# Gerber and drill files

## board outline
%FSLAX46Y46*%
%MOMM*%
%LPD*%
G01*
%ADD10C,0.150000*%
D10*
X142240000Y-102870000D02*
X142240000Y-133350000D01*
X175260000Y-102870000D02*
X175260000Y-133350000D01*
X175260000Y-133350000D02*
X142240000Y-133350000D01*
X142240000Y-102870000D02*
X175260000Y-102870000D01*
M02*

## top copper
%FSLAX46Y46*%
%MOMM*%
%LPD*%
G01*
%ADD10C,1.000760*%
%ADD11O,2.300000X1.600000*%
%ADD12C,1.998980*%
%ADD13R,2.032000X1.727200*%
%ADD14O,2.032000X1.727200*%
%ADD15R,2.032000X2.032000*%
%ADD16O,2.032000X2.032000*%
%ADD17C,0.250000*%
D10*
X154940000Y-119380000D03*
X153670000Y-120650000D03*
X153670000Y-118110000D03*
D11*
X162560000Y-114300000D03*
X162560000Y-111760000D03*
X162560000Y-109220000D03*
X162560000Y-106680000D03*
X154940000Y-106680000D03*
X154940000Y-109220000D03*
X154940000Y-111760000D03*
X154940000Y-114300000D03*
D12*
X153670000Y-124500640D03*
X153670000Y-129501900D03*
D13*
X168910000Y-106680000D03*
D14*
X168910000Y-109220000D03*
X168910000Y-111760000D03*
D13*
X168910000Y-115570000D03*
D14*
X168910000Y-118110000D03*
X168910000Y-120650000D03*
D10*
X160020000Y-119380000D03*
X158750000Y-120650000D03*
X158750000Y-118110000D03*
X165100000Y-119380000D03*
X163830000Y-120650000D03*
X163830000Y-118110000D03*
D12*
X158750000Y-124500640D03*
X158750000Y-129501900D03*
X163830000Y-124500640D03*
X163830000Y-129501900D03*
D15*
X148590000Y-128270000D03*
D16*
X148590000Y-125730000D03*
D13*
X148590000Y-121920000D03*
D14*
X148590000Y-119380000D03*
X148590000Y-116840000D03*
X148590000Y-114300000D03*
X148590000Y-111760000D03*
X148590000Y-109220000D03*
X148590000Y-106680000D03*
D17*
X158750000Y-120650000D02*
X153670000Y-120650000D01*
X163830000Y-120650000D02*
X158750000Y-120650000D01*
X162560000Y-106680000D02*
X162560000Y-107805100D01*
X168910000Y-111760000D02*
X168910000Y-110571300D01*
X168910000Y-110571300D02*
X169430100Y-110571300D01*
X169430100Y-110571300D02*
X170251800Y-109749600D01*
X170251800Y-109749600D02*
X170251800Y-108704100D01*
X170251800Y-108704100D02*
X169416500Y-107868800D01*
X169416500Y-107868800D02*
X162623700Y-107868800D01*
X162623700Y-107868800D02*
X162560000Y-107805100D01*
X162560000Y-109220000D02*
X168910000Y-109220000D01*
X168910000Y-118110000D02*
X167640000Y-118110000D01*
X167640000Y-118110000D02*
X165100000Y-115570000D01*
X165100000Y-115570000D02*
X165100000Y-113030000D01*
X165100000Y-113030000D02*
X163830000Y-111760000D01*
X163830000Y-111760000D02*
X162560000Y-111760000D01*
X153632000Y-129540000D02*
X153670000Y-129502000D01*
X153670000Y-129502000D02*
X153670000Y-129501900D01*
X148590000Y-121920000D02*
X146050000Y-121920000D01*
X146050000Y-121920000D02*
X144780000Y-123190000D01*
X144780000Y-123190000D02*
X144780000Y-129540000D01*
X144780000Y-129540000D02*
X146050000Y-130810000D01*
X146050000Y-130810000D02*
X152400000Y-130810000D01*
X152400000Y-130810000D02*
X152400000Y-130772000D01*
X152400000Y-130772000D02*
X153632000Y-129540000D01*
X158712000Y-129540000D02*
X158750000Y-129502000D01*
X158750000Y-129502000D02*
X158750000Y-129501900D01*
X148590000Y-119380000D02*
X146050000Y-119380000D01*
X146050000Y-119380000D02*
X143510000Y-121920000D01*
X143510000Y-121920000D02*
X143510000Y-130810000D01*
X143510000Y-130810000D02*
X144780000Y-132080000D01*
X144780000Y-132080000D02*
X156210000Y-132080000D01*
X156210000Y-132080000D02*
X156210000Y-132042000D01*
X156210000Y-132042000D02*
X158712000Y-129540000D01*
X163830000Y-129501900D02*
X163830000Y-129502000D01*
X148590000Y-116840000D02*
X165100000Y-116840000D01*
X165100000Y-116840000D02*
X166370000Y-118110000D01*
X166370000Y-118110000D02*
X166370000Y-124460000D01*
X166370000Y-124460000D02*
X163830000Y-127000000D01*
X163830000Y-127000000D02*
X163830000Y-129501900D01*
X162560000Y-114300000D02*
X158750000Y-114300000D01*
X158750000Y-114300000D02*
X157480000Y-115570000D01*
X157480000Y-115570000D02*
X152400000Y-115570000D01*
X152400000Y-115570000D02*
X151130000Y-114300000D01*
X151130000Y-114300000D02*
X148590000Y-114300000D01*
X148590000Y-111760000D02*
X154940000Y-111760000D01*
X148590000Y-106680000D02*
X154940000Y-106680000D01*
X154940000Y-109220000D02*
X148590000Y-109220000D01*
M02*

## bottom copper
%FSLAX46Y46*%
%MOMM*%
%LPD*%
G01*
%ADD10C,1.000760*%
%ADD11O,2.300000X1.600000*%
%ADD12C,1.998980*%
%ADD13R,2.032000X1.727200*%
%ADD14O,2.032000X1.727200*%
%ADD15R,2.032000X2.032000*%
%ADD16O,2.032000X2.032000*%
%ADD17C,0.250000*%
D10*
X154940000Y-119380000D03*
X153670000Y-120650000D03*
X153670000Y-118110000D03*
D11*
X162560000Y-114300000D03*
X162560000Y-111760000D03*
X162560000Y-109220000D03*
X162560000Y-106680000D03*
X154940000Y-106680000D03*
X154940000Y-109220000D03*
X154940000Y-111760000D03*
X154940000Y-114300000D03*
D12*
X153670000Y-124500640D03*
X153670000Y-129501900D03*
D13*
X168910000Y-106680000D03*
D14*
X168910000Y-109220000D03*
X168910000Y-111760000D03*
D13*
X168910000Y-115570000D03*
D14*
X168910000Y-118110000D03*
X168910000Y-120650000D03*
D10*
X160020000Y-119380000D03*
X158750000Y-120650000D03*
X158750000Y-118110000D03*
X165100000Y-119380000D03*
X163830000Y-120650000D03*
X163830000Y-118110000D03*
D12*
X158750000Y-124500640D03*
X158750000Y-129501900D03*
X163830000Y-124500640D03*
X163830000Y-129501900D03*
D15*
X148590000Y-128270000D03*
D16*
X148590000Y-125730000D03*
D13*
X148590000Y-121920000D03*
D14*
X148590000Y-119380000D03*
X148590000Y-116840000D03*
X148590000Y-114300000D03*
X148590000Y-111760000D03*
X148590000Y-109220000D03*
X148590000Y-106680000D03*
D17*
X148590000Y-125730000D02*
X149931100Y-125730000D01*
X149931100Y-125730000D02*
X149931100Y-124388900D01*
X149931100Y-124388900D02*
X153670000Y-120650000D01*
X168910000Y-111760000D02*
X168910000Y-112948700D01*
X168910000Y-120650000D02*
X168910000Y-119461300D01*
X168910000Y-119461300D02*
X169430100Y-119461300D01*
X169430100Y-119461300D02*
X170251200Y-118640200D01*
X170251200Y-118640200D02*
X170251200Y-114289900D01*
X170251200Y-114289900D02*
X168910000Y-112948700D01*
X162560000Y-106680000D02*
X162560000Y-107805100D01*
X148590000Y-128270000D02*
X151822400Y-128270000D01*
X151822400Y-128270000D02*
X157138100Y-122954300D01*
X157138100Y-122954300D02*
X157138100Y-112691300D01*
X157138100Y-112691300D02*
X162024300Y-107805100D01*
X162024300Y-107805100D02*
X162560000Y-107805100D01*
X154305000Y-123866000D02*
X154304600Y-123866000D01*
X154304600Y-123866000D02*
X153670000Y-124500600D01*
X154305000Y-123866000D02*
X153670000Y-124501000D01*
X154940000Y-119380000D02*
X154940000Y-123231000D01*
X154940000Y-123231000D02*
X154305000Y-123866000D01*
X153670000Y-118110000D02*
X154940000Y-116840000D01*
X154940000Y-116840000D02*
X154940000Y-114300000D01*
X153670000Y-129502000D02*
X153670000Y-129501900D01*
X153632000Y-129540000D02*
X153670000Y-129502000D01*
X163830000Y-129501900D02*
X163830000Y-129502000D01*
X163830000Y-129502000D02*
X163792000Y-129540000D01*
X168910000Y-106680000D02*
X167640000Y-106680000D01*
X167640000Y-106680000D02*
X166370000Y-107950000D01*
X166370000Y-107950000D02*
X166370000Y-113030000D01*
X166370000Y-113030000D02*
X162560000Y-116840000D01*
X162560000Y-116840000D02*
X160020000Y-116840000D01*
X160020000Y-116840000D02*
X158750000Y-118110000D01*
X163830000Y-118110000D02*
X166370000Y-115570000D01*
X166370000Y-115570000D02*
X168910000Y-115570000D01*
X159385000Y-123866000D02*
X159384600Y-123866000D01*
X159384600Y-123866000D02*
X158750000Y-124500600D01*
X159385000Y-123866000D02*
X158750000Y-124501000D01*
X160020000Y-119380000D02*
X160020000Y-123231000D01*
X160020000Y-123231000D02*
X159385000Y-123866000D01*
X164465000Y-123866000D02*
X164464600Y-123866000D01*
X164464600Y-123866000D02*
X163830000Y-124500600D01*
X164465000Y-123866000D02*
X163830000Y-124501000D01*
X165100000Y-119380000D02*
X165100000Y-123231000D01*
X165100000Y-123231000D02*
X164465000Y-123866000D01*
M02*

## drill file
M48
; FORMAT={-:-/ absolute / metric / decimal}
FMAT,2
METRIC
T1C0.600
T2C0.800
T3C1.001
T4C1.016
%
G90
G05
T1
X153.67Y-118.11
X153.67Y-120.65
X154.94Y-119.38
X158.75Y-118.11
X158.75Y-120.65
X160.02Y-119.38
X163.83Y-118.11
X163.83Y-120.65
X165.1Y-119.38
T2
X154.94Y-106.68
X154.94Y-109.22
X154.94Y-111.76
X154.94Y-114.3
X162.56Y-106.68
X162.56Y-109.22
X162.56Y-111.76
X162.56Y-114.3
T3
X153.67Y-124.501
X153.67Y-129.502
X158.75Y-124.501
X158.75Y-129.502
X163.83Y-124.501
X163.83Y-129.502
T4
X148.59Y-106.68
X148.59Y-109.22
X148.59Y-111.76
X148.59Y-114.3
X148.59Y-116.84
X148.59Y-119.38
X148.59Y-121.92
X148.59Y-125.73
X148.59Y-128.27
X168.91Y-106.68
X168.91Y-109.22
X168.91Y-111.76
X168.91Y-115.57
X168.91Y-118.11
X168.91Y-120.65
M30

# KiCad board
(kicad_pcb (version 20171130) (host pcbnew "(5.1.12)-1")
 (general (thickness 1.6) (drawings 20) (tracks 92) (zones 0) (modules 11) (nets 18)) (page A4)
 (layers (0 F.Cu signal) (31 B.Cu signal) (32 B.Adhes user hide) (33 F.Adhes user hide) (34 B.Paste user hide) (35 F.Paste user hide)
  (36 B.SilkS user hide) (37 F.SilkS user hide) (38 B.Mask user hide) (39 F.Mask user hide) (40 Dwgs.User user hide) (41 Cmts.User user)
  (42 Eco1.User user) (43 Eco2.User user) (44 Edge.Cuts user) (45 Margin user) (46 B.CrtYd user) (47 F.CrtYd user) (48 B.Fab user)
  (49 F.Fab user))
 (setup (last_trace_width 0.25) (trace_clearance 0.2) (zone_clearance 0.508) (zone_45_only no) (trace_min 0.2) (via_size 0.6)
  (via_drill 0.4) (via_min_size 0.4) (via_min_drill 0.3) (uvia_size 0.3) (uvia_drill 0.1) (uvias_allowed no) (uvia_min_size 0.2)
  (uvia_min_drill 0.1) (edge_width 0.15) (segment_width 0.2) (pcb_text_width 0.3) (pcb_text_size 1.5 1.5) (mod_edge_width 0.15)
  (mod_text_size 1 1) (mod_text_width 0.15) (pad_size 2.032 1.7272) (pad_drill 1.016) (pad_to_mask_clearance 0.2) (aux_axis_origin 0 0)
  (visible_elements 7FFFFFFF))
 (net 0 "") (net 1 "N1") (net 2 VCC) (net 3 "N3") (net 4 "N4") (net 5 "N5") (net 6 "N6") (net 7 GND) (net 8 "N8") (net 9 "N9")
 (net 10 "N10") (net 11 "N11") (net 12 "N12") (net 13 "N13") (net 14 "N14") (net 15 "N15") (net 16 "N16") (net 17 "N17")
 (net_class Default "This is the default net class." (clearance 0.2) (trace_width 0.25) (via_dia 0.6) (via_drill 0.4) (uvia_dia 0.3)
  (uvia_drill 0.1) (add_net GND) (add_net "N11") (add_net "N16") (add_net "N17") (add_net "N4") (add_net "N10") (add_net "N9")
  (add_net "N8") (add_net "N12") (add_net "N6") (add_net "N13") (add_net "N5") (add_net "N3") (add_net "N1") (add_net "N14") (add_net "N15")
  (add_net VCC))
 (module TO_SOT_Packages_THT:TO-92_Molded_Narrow (layer F.Cu) (at 153.67 118.11 270)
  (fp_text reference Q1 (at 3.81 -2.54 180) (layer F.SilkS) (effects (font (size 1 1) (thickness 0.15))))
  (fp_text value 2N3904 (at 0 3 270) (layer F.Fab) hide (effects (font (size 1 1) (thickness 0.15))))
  (pad 2 thru_hole circle (at 1.27 -1.27) (size 1.00076 1.00076) (drill 0.6) (layers *.Cu *.Mask F.SilkS) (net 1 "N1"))
  (pad 3 thru_hole circle (at 2.54 0) (size 1.00076 1.00076) (drill 0.6) (layers *.Cu *.Mask F.SilkS) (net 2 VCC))
  (pad 1 thru_hole circle (at 0 0) (size 1.00076 1.00076) (drill 0.6) (layers *.Cu *.Mask F.SilkS) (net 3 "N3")))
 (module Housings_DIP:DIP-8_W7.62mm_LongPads (layer F.Cu) (at 162.56 114.3 180)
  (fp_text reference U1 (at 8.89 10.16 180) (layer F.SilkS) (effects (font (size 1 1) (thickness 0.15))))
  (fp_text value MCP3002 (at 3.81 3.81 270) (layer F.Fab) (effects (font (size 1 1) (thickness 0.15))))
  (pad 1 thru_hole oval (at 0 0 180) (size 2.3 1.6) (drill 0.8) (layers *.Cu *.Mask F.SilkS) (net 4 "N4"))
  (pad 2 thru_hole oval (at 0 2.54 180) (size 2.3 1.6) (drill 0.8) (layers *.Cu *.Mask F.SilkS) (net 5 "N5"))
  (pad 3 thru_hole oval (at 0 5.08 180) (size 2.3 1.6) (drill 0.8) (layers *.Cu *.Mask F.SilkS) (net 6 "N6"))
  (pad 4 thru_hole oval (at 0 7.62 180) (size 2.3 1.6) (drill 0.8) (layers *.Cu *.Mask F.SilkS) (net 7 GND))
  (pad 5 thru_hole oval (at 7.62 7.62 180) (size 2.3 1.6) (drill 0.8) (layers *.Cu *.Mask F.SilkS) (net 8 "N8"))
  (pad 6 thru_hole oval (at 7.62 5.08 180) (size 2.3 1.6) (drill 0.8) (layers *.Cu *.Mask F.SilkS) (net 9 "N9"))
  (pad 7 thru_hole oval (at 7.62 2.54 180) (size 2.3 1.6) (drill 0.8) (layers *.Cu *.Mask F.SilkS) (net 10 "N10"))
  (pad 8 thru_hole oval (at 7.62 0 180) (size 2.3 1.6) (drill 0.8) (layers *.Cu *.Mask F.SilkS) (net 3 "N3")))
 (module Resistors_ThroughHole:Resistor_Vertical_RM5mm (layer F.Cu) (at 153.67 127 270)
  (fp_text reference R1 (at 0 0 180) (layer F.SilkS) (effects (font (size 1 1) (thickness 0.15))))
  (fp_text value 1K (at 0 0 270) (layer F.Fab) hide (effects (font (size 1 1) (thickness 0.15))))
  (pad 1 thru_hole circle (at -2.49936 0 270) (size 1.99898 1.99898) (drill 1.00076) (layers *.Cu *.SilkS *.Mask) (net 1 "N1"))
  (pad 2 thru_hole circle (at 2.5019 0 270) (size 1.99898 1.99898) (drill 1.00076) (layers *.Cu *.SilkS *.Mask) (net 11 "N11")))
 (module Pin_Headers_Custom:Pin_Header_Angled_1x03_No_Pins (layer F.Cu) (at 168.91 106.68)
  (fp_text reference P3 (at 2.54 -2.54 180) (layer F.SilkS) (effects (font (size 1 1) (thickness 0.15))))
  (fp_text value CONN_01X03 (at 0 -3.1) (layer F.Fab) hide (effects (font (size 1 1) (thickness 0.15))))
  (pad 1 thru_hole rect (at 0 0) (size 2.032 1.7272) (drill 1.016) (layers *.Cu *.Mask F.SilkS) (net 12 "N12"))
  (pad 2 thru_hole oval (at 0 2.54) (size 2.032 1.7272) (drill 1.016) (layers *.Cu *.Mask F.SilkS) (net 6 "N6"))
  (pad 3 thru_hole oval (at 0 5.08) (size 2.032 1.7272) (drill 1.016) (layers *.Cu *.Mask F.SilkS) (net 7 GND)))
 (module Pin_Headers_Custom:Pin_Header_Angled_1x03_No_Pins (layer F.Cu) (at 168.91 115.57)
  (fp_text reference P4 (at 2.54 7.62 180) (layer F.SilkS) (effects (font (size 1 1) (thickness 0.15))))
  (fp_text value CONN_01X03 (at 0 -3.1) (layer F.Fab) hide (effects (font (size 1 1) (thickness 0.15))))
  (pad 1 thru_hole rect (at 0 0) (size 2.032 1.7272) (drill 1.016) (layers *.Cu *.Mask F.SilkS) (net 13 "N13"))
  (pad 2 thru_hole oval (at 0 2.54) (size 2.032 1.7272) (drill 1.016) (layers *.Cu *.Mask F.SilkS) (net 5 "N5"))
  (pad 3 thru_hole oval (at 0 5.08) (size 2.032 1.7272) (drill 1.016) (layers *.Cu *.Mask F.SilkS) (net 7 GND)))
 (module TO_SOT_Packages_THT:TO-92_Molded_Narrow (layer F.Cu) (at 158.75 118.11 270)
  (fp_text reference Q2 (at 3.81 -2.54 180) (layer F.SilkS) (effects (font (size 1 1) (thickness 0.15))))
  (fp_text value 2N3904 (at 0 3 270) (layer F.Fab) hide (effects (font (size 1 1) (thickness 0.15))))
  (pad 2 thru_hole circle (at 1.27 -1.27) (size 1.00076 1.00076) (drill 0.6) (layers *.Cu *.Mask F.SilkS) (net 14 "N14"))
  (pad 3 thru_hole circle (at 2.54 0) (size 1.00076 1.00076) (drill 0.6) (layers *.Cu *.Mask F.SilkS) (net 2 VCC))
  (pad 1 thru_hole circle (at 0 0) (size 1.00076 1.00076) (drill 0.6) (layers *.Cu *.Mask F.SilkS) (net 12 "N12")))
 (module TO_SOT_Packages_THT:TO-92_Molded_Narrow (layer F.Cu) (at 163.83 118.11 270)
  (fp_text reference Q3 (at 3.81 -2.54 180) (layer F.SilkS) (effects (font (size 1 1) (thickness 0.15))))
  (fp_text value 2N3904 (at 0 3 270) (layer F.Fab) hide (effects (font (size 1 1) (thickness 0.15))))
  (pad 2 thru_hole circle (at 1.27 -1.27) (size 1.00076 1.00076) (drill 0.6) (layers *.Cu *.Mask F.SilkS) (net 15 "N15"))
  (pad 3 thru_hole circle (at 2.54 0) (size 1.00076 1.00076) (drill 0.6) (layers *.Cu *.Mask F.SilkS) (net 2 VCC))
  (pad 1 thru_hole circle (at 0 0) (size 1.00076 1.00076) (drill 0.6) (layers *.Cu *.Mask F.SilkS) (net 13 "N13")))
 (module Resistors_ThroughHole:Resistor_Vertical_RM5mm (layer F.Cu) (at 158.75 127 270)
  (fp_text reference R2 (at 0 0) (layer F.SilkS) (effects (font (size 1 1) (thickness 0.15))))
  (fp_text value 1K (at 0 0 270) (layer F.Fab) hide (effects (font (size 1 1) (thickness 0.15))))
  (pad 1 thru_hole circle (at -2.49936 0 270) (size 1.99898 1.99898) (drill 1.00076) (layers *.Cu *.SilkS *.Mask) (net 14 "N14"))
  (pad 2 thru_hole circle (at 2.5019 0 270) (size 1.99898 1.99898) (drill 1.00076) (layers *.Cu *.SilkS *.Mask) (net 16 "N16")))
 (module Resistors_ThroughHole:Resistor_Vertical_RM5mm (layer F.Cu) (at 163.83 127 270)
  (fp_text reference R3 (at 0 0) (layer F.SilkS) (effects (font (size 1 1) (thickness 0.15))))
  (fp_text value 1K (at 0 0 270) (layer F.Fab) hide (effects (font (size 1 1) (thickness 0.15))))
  (pad 1 thru_hole circle (at -2.49936 0 270) (size 1.99898 1.99898) (drill 1.00076) (layers *.Cu *.SilkS *.Mask) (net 15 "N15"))
  (pad 2 thru_hole circle (at 2.5019 0 270) (size 1.99898 1.99898) (drill 1.00076) (layers *.Cu *.SilkS *.Mask) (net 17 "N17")))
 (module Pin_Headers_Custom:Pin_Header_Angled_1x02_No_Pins (layer F.Cu) (at 148.59 128.27 180)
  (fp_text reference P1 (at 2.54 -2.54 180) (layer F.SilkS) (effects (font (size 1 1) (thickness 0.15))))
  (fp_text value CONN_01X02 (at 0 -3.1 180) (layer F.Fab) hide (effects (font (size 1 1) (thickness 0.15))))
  (pad 1 thru_hole rect (at 0 0 180) (size 2.032 2.032) (drill 1.016) (layers *.Cu *.Mask F.SilkS) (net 7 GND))
  (pad 2 thru_hole oval (at 0 2.54 180) (size 2.032 2.032) (drill 1.016) (layers *.Cu *.Mask F.SilkS) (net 2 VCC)))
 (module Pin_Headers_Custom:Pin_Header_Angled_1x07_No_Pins (layer F.Cu) (at 148.59 121.92 180)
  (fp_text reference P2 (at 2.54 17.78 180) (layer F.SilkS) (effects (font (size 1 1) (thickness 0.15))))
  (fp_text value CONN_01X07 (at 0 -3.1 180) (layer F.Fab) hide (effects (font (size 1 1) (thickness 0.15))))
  (pad 1 thru_hole rect (at 0 0 180) (size 2.032 1.7272) (drill 1.016) (layers *.Cu *.Mask F.SilkS) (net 11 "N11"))
  (pad 2 thru_hole oval (at 0 2.54 180) (size 2.032 1.7272) (drill 1.016) (layers *.Cu *.Mask F.SilkS) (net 16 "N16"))
  (pad 3 thru_hole oval (at 0 5.08 180) (size 2.032 1.7272) (drill 1.016) (layers *.Cu *.Mask F.SilkS) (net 17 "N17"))
  (pad 4 thru_hole oval (at 0 7.62 180) (size 2.032 1.7272) (drill 1.016) (layers *.Cu *.Mask F.SilkS) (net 4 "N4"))
  (pad 5 thru_hole oval (at 0 10.16 180) (size 2.032 1.7272) (drill 1.016) (layers *.Cu *.Mask F.SilkS) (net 10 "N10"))
  (pad 6 thru_hole oval (at 0 12.7 180) (size 2.032 1.7272) (drill 1.016) (layers *.Cu *.Mask F.SilkS) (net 9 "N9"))
  (pad 7 thru_hole oval (at 0 15.24 180) (size 2.032 1.7272) (drill 1.016) (layers *.Cu *.Mask F.SilkS) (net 8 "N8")))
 (gr_line (start 142.24 102.87) (end 142.24 133.35) (angle 90) (layer Edge.Cuts) (width 0.15))
 (gr_line (start 175.26 102.87) (end 175.26 133.35) (angle 90) (layer Edge.Cuts) (width 0.15))
 (gr_line (start 175.26 133.35) (end 142.24 133.35) (angle 90) (layer Edge.Cuts) (width 0.15))
 (gr_line (start 142.24 102.87) (end 175.26 102.87) (angle 90) (layer Edge.Cuts) (width 0.15))
 (segment (start 158.75 120.65) (end 153.67 120.65) (width 0.25) (layer F.Cu) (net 2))
 (segment (start 163.83 120.65) (end 158.75 120.65) (width 0.25) (layer F.Cu) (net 2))
 (segment (start 148.59 125.73) (end 149.9311 125.73) (width 0.25) (layer B.Cu) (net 2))
 (segment (start 149.9311 125.73) (end 149.9311 124.3889) (width 0.25) (layer B.Cu) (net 2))
 (segment (start 149.9311 124.3889) (end 153.67 120.65) (width 0.25) (layer B.Cu) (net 2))
 (segment (start 162.56 106.68) (end 162.56 107.8051) (width 0.25) (layer F.Cu) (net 7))
 (segment (start 168.91 111.76) (end 168.91 110.5713) (width 0.25) (layer F.Cu) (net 7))
 (segment (start 168.91 110.5713) (end 169.4301 110.5713) (width 0.25) (layer F.Cu) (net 7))
 (segment (start 169.4301 110.5713) (end 170.2518 109.7496) (width 0.25) (layer F.Cu) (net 7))
 (segment (start 170.2518 109.7496) (end 170.2518 108.7041) (width 0.25) (layer F.Cu) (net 7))
 (segment (start 170.2518 108.7041) (end 169.4165 107.8688) (width 0.25) (layer F.Cu) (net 7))
 (segment (start 169.4165 107.8688) (end 162.6237 107.8688) (width 0.25) (layer F.Cu) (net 7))
 (segment (start 162.6237 107.8688) (end 162.56 107.8051) (width 0.25) (layer F.Cu) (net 7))
 (segment (start 168.91 111.76) (end 168.91 112.9487) (width 0.25) (layer B.Cu) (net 7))
 (segment (start 168.91 120.65) (end 168.91 119.4613) (width 0.25) (layer B.Cu) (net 7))
 (segment (start 168.91 119.4613) (end 169.4301 119.4613) (width 0.25) (layer B.Cu) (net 7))
 (segment (start 169.4301 119.4613) (end 170.2512 118.6402) (width 0.25) (layer B.Cu) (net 7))
 (segment (start 170.2512 118.6402) (end 170.2512 114.2899) (width 0.25) (layer B.Cu) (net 7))
 (segment (start 170.2512 114.2899) (end 168.91 112.9487) (width 0.25) (layer B.Cu) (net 7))
 (segment (start 162.56 106.68) (end 162.56 107.8051) (width 0.25) (layer B.Cu) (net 7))
 (segment (start 148.59 128.27) (end 151.8224 128.27) (width 0.25) (layer B.Cu) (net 7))
 (segment (start 151.8224 128.27) (end 157.1381 122.9543) (width 0.25) (layer B.Cu) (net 7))
 (segment (start 157.1381 122.9543) (end 157.1381 112.6913) (width 0.25) (layer B.Cu) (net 7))
 (segment (start 157.1381 112.6913) (end 162.0243 107.8051) (width 0.25) (layer B.Cu) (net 7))
 (segment (start 162.0243 107.8051) (end 162.56 107.8051) (width 0.25) (layer B.Cu) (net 7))
 (segment (start 162.56 109.22) (end 168.91 109.22) (width 0.25) (layer F.Cu) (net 6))
 (segment (start 168.91 118.11) (end 167.64 118.11) (width 0.25) (layer F.Cu) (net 5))
 (segment (start 167.64 118.11) (end 165.1 115.57) (width 0.25) (layer F.Cu) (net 5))
 (segment (start 165.1 115.57) (end 165.1 113.03) (width 0.25) (layer F.Cu) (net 5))
 (segment (start 165.1 113.03) (end 163.83 111.76) (width 0.25) (layer F.Cu) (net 5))
 (segment (start 163.83 111.76) (end 162.56 111.76) (width 0.25) (layer F.Cu) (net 5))
 (segment (start 154.305 123.866) (end 154.3046 123.866) (width 0.25) (layer B.Cu) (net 1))
 (segment (start 154.3046 123.866) (end 153.67 124.5006) (width 0.25) (layer B.Cu) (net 1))
 (segment (start 154.305 123.866) (end 153.67 124.501) (width 0.25) (layer B.Cu) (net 1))
 (segment (start 154.94 119.38) (end 154.94 123.231) (width 0.25) (layer B.Cu) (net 1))
 (segment (start 154.94 123.231) (end 154.305 123.866) (width 0.25) (layer B.Cu) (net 1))
 (segment (start 153.67 118.11) (end 154.94 116.84) (width 0.25) (layer B.Cu) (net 3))
 (segment (start 154.94 116.84) (end 154.94 114.3) (width 0.25) (layer B.Cu) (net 3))
 (segment (start 153.67 129.502) (end 153.67 129.5019) (width 0.25) (layer B.Cu) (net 11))
 (segment (start 153.632 129.54) (end 153.67 129.502) (width 0.25) (layer B.Cu) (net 11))
 (segment (start 153.632 129.54) (end 153.67 129.502) (width 0.25) (layer F.Cu) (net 11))
 (segment (start 153.67 129.502) (end 153.67 129.5019) (width 0.25) (layer F.Cu) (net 11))
 (segment (start 148.59 121.92) (end 146.05 121.92) (width 0.25) (layer F.Cu) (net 11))
 (segment (start 146.05 121.92) (end 144.78 123.19) (width 0.25) (layer F.Cu) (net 11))
 (segment (start 144.78 123.19) (end 144.78 129.54) (width 0.25) (layer F.Cu) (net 11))
 (segment (start 144.78 129.54) (end 146.05 130.81) (width 0.25) (layer F.Cu) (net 11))
 (segment (start 146.05 130.81) (end 152.4 130.81) (width 0.25) (layer F.Cu) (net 11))
 (segment (start 152.4 130.81) (end 152.4 130.772) (width 0.25) (layer F.Cu) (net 11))
 (segment (start 152.4 130.772) (end 153.632 129.54) (width 0.25) (layer F.Cu) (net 11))
 (segment (start 158.712 129.54) (end 158.75 129.502) (width 0.25) (layer F.Cu) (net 16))
 (segment (start 158.75 129.502) (end 158.75 129.5019) (width 0.25) (layer F.Cu) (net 16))
 (segment (start 148.59 119.38) (end 146.05 119.38) (width 0.25) (layer F.Cu) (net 16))
 (segment (start 146.05 119.38) (end 143.51 121.92) (width 0.25) (layer F.Cu) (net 16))
 (segment (start 143.51 121.92) (end 143.51 130.81) (width 0.25) (layer F.Cu) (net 16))
 (segment (start 143.51 130.81) (end 144.78 132.08) (width 0.25) (layer F.Cu) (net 16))
 (segment (start 144.78 132.08) (end 156.21 132.08) (width 0.25) (layer F.Cu) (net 16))
 (segment (start 156.21 132.08) (end 156.21 132.042) (width 0.25) (layer F.Cu) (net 16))
 (segment (start 156.21 132.042) (end 158.712 129.54) (width 0.25) (layer F.Cu) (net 16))
 (segment (start 163.83 129.5019) (end 163.83 129.502) (width 0.25) (layer B.Cu) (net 17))
 (segment (start 163.83 129.5019) (end 163.83 129.502) (width 0.25) (layer F.Cu) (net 17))
 (segment (start 148.59 116.84) (end 165.1 116.84) (width 0.25) (layer F.Cu) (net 17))
 (segment (start 165.1 116.84) (end 166.37 118.11) (width 0.25) (layer F.Cu) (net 17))
 (segment (start 166.37 118.11) (end 166.37 124.46) (width 0.25) (layer F.Cu) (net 17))
 (segment (start 166.37 124.46) (end 163.83 127) (width 0.25) (layer F.Cu) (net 17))
 (segment (start 163.83 127) (end 163.83 129.5019) (width 0.25) (layer F.Cu) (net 17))
 (segment (start 163.83 129.502) (end 163.792 129.54) (width 0.25) (layer B.Cu) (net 17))
 (segment (start 162.56 114.3) (end 158.75 114.3) (width 0.25) (layer F.Cu) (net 4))
 (segment (start 158.75 114.3) (end 157.48 115.57) (width 0.25) (layer F.Cu) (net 4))
 (segment (start 157.48 115.57) (end 152.4 115.57) (width 0.25) (layer F.Cu) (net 4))
 (segment (start 152.4 115.57) (end 151.13 114.3) (width 0.25) (layer F.Cu) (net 4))
 (segment (start 151.13 114.3) (end 148.59 114.3) (width 0.25) (layer F.Cu) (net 4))
 (segment (start 148.59 111.76) (end 154.94 111.76) (width 0.25) (layer F.Cu) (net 10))
 (segment (start 168.91 106.68) (end 167.64 106.68) (width 0.25) (layer B.Cu) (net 12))
 (segment (start 167.64 106.68) (end 166.37 107.95) (width 0.25) (layer B.Cu) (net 12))
 (segment (start 166.37 107.95) (end 166.37 113.03) (width 0.25) (layer B.Cu) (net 12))
 (segment (start 166.37 113.03) (end 162.56 116.84) (width 0.25) (layer B.Cu) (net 12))
 (segment (start 162.56 116.84) (end 160.02 116.84) (width 0.25) (layer B.Cu) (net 12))
 (segment (start 160.02 116.84) (end 158.75 118.11) (width 0.25) (layer B.Cu) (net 12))
 (segment (start 163.83 118.11) (end 166.37 115.57) (width 0.25) (layer B.Cu) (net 13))
 (segment (start 166.37 115.57) (end 168.91 115.57) (width 0.25) (layer B.Cu) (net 13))
 (segment (start 159.385 123.866) (end 159.3846 123.866) (width 0.25) (layer B.Cu) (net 14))
 (segment (start 159.3846 123.866) (end 158.75 124.5006) (width 0.25) (layer B.Cu) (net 14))
 (segment (start 159.385 123.866) (end 158.75 124.501) (width 0.25) (layer B.Cu) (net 14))
 (segment (start 160.02 119.38) (end 160.02 123.231) (width 0.25) (layer B.Cu) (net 14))
 (segment (start 160.02 123.231) (end 159.385 123.866) (width 0.25) (layer B.Cu) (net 14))
 (segment (start 164.465 123.866) (end 164.4646 123.866) (width 0.25) (layer B.Cu) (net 15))
 (segment (start 164.4646 123.866) (end 163.83 124.5006) (width 0.25) (layer B.Cu) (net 15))
 (segment (start 164.465 123.866) (end 163.83 124.501) (width 0.25) (layer B.Cu) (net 15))
 (segment (start 165.1 119.38) (end 165.1 123.231) (width 0.25) (layer B.Cu) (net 15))
 (segment (start 165.1 123.231) (end 164.465 123.866) (width 0.25) (layer B.Cu) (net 15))
 (segment (start 148.59 106.68) (end 154.94 106.68) (width 0.25) (layer F.Cu) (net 8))
 (segment (start 154.94 109.22) (end 148.59 109.22) (width 0.25) (layer F.Cu) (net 9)))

